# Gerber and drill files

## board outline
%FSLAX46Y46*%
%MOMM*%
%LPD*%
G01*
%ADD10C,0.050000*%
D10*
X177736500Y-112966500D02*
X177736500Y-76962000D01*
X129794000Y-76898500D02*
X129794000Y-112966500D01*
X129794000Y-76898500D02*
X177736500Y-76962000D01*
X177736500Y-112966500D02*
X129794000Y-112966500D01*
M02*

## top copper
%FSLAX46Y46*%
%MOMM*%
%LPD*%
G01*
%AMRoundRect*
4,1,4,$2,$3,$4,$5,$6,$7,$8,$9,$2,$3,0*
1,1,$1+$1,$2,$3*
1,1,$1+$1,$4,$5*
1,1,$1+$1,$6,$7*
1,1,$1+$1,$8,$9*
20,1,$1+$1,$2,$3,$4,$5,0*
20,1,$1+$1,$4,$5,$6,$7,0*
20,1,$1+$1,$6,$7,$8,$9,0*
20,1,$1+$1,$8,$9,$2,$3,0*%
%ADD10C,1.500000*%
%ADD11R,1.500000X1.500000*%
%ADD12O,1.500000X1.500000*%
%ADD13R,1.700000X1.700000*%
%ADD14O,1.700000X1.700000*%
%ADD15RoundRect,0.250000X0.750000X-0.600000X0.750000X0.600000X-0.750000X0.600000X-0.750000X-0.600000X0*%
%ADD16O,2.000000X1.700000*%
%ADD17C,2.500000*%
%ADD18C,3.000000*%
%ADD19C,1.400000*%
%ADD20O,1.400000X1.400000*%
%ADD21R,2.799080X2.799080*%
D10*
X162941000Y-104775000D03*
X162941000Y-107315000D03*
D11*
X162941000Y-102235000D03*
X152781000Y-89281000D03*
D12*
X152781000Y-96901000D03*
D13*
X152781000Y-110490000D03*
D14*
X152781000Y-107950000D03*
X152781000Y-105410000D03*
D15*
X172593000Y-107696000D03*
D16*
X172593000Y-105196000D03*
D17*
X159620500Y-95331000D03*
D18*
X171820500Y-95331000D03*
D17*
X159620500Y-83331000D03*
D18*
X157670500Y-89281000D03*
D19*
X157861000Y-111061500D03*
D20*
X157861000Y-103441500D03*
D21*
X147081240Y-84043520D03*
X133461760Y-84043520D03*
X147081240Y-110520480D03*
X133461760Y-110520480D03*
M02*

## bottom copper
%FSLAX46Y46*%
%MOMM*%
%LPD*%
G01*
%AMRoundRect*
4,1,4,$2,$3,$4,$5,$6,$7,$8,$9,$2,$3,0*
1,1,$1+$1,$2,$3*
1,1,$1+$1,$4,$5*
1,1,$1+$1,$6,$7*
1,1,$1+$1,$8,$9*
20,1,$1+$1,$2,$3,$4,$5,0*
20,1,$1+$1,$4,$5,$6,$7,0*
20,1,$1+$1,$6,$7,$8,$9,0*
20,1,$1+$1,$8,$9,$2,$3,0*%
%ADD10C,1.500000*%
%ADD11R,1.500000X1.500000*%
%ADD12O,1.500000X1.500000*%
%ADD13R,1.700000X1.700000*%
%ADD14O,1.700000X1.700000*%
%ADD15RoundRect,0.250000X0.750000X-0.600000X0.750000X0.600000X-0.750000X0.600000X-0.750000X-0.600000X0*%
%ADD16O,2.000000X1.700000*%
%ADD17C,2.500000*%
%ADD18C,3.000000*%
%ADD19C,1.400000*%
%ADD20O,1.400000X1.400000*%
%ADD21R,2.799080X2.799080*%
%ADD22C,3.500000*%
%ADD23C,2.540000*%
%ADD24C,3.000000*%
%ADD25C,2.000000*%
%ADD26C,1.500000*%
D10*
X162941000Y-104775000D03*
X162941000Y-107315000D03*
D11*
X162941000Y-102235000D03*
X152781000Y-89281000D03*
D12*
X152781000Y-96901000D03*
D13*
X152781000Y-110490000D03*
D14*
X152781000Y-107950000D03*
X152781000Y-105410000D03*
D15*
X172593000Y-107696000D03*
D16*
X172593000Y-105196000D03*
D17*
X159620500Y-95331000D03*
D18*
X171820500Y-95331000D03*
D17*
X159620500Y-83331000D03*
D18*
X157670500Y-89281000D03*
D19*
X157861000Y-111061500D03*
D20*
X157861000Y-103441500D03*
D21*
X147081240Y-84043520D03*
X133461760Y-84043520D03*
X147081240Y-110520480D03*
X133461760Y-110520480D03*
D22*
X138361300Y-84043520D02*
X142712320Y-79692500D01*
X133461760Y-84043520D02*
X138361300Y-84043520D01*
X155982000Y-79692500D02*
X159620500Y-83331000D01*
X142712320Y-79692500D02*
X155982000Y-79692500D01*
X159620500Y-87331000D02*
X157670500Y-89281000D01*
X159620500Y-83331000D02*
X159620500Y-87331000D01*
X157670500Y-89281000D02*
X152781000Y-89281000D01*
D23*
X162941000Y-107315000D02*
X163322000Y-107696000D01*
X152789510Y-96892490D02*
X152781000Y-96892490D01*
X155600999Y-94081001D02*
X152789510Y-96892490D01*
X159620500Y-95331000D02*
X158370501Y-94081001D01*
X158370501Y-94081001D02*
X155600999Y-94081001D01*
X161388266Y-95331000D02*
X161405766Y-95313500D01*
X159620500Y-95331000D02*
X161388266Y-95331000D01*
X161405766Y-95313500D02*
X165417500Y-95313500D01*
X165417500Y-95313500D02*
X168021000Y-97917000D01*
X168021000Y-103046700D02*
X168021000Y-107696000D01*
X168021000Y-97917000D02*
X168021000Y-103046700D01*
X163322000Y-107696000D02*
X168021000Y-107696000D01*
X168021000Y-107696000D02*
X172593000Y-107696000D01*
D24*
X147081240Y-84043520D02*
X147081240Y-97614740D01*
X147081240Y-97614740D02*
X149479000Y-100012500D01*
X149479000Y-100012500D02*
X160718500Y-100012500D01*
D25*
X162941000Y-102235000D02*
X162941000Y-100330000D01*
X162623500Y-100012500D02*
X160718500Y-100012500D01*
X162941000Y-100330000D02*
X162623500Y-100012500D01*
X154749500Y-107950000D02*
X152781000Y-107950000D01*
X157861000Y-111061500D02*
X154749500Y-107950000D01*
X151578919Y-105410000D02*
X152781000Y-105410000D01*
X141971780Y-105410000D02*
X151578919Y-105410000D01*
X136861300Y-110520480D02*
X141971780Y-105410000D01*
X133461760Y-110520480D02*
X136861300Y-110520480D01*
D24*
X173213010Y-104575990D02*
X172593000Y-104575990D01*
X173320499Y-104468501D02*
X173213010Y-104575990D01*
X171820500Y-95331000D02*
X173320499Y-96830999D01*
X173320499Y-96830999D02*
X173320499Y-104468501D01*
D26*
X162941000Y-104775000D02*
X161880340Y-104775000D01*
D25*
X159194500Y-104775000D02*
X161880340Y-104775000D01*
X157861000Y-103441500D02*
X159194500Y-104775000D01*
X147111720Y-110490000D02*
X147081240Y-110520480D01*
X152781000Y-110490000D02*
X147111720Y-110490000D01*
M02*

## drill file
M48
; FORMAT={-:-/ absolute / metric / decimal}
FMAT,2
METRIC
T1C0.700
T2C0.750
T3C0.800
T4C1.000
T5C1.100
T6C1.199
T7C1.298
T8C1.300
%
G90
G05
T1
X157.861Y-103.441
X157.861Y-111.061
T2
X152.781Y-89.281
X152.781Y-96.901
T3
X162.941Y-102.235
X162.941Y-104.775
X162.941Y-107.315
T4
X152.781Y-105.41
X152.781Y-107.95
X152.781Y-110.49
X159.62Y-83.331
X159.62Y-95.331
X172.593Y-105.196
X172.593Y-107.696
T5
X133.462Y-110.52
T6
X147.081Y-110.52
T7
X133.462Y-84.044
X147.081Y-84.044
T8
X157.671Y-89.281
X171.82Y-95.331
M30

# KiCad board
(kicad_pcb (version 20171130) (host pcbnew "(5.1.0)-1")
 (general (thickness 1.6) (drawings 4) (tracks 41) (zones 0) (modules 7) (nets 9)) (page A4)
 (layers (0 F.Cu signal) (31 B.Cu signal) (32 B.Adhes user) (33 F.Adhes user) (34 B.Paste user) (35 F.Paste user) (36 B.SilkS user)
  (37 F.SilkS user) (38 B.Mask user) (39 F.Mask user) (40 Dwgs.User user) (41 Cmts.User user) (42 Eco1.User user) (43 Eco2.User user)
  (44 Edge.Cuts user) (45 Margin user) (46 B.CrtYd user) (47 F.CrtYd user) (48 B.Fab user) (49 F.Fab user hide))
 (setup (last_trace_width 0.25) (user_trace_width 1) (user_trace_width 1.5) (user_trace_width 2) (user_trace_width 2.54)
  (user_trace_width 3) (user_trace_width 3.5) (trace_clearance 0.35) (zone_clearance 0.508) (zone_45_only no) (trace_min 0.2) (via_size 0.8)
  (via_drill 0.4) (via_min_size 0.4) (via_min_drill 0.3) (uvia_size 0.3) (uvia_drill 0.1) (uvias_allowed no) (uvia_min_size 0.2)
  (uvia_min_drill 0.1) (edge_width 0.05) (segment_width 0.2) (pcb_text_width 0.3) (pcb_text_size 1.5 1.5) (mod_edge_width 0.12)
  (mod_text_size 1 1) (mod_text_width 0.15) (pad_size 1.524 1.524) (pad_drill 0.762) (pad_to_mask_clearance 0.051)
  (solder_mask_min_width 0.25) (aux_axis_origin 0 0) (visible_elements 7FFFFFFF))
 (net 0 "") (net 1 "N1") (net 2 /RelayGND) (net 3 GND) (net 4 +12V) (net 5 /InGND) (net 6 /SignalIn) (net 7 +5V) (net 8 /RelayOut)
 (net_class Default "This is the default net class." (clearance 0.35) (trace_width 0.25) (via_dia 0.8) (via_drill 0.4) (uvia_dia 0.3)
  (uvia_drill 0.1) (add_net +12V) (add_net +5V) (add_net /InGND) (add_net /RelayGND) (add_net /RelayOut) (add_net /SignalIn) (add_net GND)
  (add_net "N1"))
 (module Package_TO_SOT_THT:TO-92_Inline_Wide (layer F.Cu) (at 162.941 102.235 270)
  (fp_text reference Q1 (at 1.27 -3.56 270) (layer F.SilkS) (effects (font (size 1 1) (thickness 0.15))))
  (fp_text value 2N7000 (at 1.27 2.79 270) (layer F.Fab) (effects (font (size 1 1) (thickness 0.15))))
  (pad 2 thru_hole circle (at 2.54 0) (size 1.5 1.5) (drill 0.8) (layers *.Cu *.Mask) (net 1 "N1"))
  (pad 3 thru_hole circle (at 5.08 0) (size 1.5 1.5) (drill 0.8) (layers *.Cu *.Mask) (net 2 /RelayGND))
  (pad 1 thru_hole rect (at 0 0) (size 1.5 1.5) (drill 0.8) (layers *.Cu *.Mask) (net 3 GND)))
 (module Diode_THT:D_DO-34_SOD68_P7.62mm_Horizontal (layer F.Cu) (at 152.781 89.281 270)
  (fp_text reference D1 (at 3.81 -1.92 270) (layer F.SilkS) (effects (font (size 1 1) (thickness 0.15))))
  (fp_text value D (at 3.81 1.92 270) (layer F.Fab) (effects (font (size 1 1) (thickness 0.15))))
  (pad 1 thru_hole rect (at 0 0 270) (size 1.5 1.5) (drill 0.75) (layers *.Cu *.Mask) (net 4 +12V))
  (pad 2 thru_hole oval (at 7.62 0 270) (size 1.5 1.5) (drill 0.75) (layers *.Cu *.Mask) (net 2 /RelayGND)))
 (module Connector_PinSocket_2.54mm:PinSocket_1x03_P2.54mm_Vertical (layer F.Cu) (at 152.781 110.49 180)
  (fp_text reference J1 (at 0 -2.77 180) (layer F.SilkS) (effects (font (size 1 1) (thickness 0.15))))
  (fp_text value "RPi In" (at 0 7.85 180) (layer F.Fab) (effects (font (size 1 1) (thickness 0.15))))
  (pad 1 thru_hole rect (at 0 0 180) (size 1.7 1.7) (drill 1) (layers *.Cu *.Mask) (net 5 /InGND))
  (pad 2 thru_hole oval (at 0 2.54 180) (size 1.7 1.7) (drill 1) (layers *.Cu *.Mask) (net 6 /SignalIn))
  (pad 3 thru_hole oval (at 0 5.08 180) (size 1.7 1.7) (drill 1) (layers *.Cu *.Mask) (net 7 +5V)))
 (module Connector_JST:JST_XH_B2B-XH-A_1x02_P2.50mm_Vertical (layer F.Cu) (at 172.593 107.696 90)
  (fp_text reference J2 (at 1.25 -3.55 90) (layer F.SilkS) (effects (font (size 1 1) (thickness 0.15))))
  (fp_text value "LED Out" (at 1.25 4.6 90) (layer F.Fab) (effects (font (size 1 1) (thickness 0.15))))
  (pad 1 thru_hole roundrect (at 0 0 90) (size 1.7 2) (drill 1) (layers *.Cu *.Mask) (roundrect_rratio 0.147059) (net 2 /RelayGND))
  (pad 2 thru_hole oval (at 2.5 0 90) (size 1.7 2) (drill 1) (layers *.Cu *.Mask) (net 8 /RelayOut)))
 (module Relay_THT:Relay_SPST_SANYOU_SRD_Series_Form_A (layer F.Cu) (at 157.6705 89.281)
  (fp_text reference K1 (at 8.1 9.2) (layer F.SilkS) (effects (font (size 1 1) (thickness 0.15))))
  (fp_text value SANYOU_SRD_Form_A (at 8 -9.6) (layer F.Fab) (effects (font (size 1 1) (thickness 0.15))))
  (pad 2 thru_hole circle (at 1.95 6.05 90) (size 2.5 2.5) (drill 1) (layers *.Cu *.Mask) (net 2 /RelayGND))
  (pad 3 thru_hole circle (at 14.15 6.05 90) (size 3 3) (drill 1.3) (layers *.Cu *.Mask) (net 8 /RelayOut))
  (pad 5 thru_hole circle (at 1.95 -5.95 90) (size 2.5 2.5) (drill 1) (layers *.Cu *.Mask) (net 4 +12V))
  (pad 1 thru_hole circle (at 0 0 90) (size 3 3) (drill 1.3) (layers *.Cu *.Mask) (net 4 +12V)))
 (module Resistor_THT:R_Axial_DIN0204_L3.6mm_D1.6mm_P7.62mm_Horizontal (layer F.Cu) (at 157.861 111.0615 90)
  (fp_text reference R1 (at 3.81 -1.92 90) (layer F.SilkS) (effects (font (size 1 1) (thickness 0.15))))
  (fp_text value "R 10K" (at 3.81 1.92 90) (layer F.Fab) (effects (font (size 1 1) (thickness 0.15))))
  (pad 1 thru_hole circle (at 0 0 90) (size 1.4 1.4) (drill 0.7) (layers *.Cu *.Mask) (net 6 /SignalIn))
  (pad 2 thru_hole oval (at 7.62 0 90) (size 1.4 1.4) (drill 0.7) (layers *.Cu *.Mask) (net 1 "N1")))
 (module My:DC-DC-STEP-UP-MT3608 (layer F.Cu) (at 140.2715 97.282 90)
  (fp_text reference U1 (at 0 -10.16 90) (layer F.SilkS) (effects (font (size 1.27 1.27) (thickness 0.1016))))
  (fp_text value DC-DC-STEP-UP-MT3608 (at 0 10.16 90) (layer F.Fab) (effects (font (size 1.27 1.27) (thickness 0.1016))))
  (pad OUT- thru_hole rect (at 13.23848 6.80974 90) (size 2.79908 2.79908) (drill 1.29794) (layers *.Cu *.Paste *.Mask) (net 3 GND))
  (pad OUT+ thru_hole rect (at 13.23848 -6.80974 90) (size 2.79908 2.79908) (drill 1.29794) (layers *.Cu *.Paste *.Mask) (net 4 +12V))
  (pad IN- thru_hole rect (at -13.23848 6.80974 90) (size 2.79908 2.79908) (drill 1.19888) (layers *.Cu *.Paste *.Mask) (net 5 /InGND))
  (pad IN+ thru_hole rect (at -13.23848 -6.80974 90) (size 2.79908 2.79908) (drill 1.09982) (layers *.Cu *.Paste *.Mask) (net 7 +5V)))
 (gr_line (start 177.7365 112.9665) (end 177.7365 76.962) (layer Edge.Cuts) (width 0.05))
 (gr_line (start 129.794 76.8985) (end 129.794 112.9665) (layer Edge.Cuts) (width 0.05))
 (gr_line (start 129.794 76.8985) (end 177.7365 76.962) (layer Edge.Cuts) (width 0.05))
 (gr_line (start 177.7365 112.9665) (end 129.794 112.9665) (layer Edge.Cuts) (width 0.05))
 (segment (start 138.3613 84.04352) (end 142.71232 79.6925) (width 3.5) (layer B.Cu) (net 4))
 (segment (start 133.46176 84.04352) (end 138.3613 84.04352) (width 3.5) (layer B.Cu) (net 4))
 (segment (start 155.982 79.6925) (end 159.6205 83.331) (width 3.5) (layer B.Cu) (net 4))
 (segment (start 142.71232 79.6925) (end 155.982 79.6925) (width 3.5) (layer B.Cu) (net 4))
 (segment (start 159.6205 87.331) (end 157.6705 89.281) (width 3.5) (layer B.Cu) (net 4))
 (segment (start 159.6205 83.331) (end 159.6205 87.331) (width 3.5) (layer B.Cu) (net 4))
 (segment (start 157.6705 89.281) (end 152.781 89.281) (width 3.5) (layer B.Cu) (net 4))
 (segment (start 162.941 107.315) (end 163.322 107.696) (width 2.54) (layer B.Cu) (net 2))
 (segment (start 152.78951 96.89249) (end 152.781 96.89249) (width 2.54) (layer B.Cu) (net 2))
 (segment (start 155.600999 94.081001) (end 152.78951 96.89249) (width 2.54) (layer B.Cu) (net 2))
 (segment (start 159.6205 95.331) (end 158.370501 94.081001) (width 2.54) (layer B.Cu) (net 2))
 (segment (start 158.370501 94.081001) (end 155.600999 94.081001) (width 2.54) (layer B.Cu) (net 2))
 (segment (start 161.388266 95.331) (end 161.405766 95.3135) (width 2.54) (layer B.Cu) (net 2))
 (segment (start 159.6205 95.331) (end 161.388266 95.331) (width 2.54) (layer B.Cu) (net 2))
 (segment (start 161.405766 95.3135) (end 165.4175 95.3135) (width 2.54) (layer B.Cu) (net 2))
 (segment (start 165.4175 95.3135) (end 168.021 97.917) (width 2.54) (layer B.Cu) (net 2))
 (segment (start 168.021 103.0467) (end 168.021 107.696) (width 2.54) (layer B.Cu) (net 2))
 (segment (start 168.021 97.917) (end 168.021 103.0467) (width 2.54) (layer B.Cu) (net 2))
 (segment (start 163.322 107.696) (end 168.021 107.696) (width 2.54) (layer B.Cu) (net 2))
 (segment (start 168.021 107.696) (end 172.593 107.696) (width 2.54) (layer B.Cu) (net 2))
 (segment (start 147.08124 84.04352) (end 147.08124 97.61474) (width 3) (layer B.Cu) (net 3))
 (segment (start 147.08124 97.61474) (end 149.479 100.0125) (width 3) (layer B.Cu) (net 3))
 (segment (start 149.479 100.0125) (end 160.7185 100.0125) (width 3) (layer B.Cu) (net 3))
 (segment (start 162.941 102.235) (end 162.941 100.33) (width 2) (layer B.Cu) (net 3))
 (segment (start 162.6235 100.0125) (end 160.7185 100.0125) (width 2) (layer B.Cu) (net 3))
 (segment (start 162.941 100.33) (end 162.6235 100.0125) (width 2) (layer B.Cu) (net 3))
 (segment (start 154.7495 107.95) (end 152.781 107.95) (width 2) (layer B.Cu) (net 6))
 (segment (start 157.861 111.0615) (end 154.7495 107.95) (width 2) (layer B.Cu) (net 6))
 (segment (start 151.578919 105.41) (end 152.781 105.41) (width 2) (layer B.Cu) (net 7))
 (segment (start 141.97178 105.41) (end 151.578919 105.41) (width 2) (layer B.Cu) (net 7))
 (segment (start 136.8613 110.52048) (end 141.97178 105.41) (width 2) (layer B.Cu) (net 7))
 (segment (start 133.46176 110.52048) (end 136.8613 110.52048) (width 2) (layer B.Cu) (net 7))
 (segment (start 173.21301 104.57599) (end 172.593 104.57599) (width 3) (layer B.Cu) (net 8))
 (segment (start 173.320499 104.468501) (end 173.21301 104.57599) (width 3) (layer B.Cu) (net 8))
 (segment (start 171.8205 95.331) (end 173.320499 96.830999) (width 3) (layer B.Cu) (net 8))
 (segment (start 173.320499 96.830999) (end 173.320499 104.468501) (width 3) (layer B.Cu) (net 8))
 (segment (start 162.941 104.775) (end 161.88034 104.775) (width 1.5) (layer B.Cu) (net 1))
 (segment (start 159.1945 104.775) (end 161.88034 104.775) (width 2) (layer B.Cu) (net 1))
 (segment (start 157.861 103.4415) (end 159.1945 104.775) (width 2) (layer B.Cu) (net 1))
 (segment (start 147.11172 110.49) (end 147.08124 110.52048) (width 2) (layer B.Cu) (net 5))
 (segment (start 152.781 110.49) (end 147.11172 110.49) (width 2) (layer B.Cu) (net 5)))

